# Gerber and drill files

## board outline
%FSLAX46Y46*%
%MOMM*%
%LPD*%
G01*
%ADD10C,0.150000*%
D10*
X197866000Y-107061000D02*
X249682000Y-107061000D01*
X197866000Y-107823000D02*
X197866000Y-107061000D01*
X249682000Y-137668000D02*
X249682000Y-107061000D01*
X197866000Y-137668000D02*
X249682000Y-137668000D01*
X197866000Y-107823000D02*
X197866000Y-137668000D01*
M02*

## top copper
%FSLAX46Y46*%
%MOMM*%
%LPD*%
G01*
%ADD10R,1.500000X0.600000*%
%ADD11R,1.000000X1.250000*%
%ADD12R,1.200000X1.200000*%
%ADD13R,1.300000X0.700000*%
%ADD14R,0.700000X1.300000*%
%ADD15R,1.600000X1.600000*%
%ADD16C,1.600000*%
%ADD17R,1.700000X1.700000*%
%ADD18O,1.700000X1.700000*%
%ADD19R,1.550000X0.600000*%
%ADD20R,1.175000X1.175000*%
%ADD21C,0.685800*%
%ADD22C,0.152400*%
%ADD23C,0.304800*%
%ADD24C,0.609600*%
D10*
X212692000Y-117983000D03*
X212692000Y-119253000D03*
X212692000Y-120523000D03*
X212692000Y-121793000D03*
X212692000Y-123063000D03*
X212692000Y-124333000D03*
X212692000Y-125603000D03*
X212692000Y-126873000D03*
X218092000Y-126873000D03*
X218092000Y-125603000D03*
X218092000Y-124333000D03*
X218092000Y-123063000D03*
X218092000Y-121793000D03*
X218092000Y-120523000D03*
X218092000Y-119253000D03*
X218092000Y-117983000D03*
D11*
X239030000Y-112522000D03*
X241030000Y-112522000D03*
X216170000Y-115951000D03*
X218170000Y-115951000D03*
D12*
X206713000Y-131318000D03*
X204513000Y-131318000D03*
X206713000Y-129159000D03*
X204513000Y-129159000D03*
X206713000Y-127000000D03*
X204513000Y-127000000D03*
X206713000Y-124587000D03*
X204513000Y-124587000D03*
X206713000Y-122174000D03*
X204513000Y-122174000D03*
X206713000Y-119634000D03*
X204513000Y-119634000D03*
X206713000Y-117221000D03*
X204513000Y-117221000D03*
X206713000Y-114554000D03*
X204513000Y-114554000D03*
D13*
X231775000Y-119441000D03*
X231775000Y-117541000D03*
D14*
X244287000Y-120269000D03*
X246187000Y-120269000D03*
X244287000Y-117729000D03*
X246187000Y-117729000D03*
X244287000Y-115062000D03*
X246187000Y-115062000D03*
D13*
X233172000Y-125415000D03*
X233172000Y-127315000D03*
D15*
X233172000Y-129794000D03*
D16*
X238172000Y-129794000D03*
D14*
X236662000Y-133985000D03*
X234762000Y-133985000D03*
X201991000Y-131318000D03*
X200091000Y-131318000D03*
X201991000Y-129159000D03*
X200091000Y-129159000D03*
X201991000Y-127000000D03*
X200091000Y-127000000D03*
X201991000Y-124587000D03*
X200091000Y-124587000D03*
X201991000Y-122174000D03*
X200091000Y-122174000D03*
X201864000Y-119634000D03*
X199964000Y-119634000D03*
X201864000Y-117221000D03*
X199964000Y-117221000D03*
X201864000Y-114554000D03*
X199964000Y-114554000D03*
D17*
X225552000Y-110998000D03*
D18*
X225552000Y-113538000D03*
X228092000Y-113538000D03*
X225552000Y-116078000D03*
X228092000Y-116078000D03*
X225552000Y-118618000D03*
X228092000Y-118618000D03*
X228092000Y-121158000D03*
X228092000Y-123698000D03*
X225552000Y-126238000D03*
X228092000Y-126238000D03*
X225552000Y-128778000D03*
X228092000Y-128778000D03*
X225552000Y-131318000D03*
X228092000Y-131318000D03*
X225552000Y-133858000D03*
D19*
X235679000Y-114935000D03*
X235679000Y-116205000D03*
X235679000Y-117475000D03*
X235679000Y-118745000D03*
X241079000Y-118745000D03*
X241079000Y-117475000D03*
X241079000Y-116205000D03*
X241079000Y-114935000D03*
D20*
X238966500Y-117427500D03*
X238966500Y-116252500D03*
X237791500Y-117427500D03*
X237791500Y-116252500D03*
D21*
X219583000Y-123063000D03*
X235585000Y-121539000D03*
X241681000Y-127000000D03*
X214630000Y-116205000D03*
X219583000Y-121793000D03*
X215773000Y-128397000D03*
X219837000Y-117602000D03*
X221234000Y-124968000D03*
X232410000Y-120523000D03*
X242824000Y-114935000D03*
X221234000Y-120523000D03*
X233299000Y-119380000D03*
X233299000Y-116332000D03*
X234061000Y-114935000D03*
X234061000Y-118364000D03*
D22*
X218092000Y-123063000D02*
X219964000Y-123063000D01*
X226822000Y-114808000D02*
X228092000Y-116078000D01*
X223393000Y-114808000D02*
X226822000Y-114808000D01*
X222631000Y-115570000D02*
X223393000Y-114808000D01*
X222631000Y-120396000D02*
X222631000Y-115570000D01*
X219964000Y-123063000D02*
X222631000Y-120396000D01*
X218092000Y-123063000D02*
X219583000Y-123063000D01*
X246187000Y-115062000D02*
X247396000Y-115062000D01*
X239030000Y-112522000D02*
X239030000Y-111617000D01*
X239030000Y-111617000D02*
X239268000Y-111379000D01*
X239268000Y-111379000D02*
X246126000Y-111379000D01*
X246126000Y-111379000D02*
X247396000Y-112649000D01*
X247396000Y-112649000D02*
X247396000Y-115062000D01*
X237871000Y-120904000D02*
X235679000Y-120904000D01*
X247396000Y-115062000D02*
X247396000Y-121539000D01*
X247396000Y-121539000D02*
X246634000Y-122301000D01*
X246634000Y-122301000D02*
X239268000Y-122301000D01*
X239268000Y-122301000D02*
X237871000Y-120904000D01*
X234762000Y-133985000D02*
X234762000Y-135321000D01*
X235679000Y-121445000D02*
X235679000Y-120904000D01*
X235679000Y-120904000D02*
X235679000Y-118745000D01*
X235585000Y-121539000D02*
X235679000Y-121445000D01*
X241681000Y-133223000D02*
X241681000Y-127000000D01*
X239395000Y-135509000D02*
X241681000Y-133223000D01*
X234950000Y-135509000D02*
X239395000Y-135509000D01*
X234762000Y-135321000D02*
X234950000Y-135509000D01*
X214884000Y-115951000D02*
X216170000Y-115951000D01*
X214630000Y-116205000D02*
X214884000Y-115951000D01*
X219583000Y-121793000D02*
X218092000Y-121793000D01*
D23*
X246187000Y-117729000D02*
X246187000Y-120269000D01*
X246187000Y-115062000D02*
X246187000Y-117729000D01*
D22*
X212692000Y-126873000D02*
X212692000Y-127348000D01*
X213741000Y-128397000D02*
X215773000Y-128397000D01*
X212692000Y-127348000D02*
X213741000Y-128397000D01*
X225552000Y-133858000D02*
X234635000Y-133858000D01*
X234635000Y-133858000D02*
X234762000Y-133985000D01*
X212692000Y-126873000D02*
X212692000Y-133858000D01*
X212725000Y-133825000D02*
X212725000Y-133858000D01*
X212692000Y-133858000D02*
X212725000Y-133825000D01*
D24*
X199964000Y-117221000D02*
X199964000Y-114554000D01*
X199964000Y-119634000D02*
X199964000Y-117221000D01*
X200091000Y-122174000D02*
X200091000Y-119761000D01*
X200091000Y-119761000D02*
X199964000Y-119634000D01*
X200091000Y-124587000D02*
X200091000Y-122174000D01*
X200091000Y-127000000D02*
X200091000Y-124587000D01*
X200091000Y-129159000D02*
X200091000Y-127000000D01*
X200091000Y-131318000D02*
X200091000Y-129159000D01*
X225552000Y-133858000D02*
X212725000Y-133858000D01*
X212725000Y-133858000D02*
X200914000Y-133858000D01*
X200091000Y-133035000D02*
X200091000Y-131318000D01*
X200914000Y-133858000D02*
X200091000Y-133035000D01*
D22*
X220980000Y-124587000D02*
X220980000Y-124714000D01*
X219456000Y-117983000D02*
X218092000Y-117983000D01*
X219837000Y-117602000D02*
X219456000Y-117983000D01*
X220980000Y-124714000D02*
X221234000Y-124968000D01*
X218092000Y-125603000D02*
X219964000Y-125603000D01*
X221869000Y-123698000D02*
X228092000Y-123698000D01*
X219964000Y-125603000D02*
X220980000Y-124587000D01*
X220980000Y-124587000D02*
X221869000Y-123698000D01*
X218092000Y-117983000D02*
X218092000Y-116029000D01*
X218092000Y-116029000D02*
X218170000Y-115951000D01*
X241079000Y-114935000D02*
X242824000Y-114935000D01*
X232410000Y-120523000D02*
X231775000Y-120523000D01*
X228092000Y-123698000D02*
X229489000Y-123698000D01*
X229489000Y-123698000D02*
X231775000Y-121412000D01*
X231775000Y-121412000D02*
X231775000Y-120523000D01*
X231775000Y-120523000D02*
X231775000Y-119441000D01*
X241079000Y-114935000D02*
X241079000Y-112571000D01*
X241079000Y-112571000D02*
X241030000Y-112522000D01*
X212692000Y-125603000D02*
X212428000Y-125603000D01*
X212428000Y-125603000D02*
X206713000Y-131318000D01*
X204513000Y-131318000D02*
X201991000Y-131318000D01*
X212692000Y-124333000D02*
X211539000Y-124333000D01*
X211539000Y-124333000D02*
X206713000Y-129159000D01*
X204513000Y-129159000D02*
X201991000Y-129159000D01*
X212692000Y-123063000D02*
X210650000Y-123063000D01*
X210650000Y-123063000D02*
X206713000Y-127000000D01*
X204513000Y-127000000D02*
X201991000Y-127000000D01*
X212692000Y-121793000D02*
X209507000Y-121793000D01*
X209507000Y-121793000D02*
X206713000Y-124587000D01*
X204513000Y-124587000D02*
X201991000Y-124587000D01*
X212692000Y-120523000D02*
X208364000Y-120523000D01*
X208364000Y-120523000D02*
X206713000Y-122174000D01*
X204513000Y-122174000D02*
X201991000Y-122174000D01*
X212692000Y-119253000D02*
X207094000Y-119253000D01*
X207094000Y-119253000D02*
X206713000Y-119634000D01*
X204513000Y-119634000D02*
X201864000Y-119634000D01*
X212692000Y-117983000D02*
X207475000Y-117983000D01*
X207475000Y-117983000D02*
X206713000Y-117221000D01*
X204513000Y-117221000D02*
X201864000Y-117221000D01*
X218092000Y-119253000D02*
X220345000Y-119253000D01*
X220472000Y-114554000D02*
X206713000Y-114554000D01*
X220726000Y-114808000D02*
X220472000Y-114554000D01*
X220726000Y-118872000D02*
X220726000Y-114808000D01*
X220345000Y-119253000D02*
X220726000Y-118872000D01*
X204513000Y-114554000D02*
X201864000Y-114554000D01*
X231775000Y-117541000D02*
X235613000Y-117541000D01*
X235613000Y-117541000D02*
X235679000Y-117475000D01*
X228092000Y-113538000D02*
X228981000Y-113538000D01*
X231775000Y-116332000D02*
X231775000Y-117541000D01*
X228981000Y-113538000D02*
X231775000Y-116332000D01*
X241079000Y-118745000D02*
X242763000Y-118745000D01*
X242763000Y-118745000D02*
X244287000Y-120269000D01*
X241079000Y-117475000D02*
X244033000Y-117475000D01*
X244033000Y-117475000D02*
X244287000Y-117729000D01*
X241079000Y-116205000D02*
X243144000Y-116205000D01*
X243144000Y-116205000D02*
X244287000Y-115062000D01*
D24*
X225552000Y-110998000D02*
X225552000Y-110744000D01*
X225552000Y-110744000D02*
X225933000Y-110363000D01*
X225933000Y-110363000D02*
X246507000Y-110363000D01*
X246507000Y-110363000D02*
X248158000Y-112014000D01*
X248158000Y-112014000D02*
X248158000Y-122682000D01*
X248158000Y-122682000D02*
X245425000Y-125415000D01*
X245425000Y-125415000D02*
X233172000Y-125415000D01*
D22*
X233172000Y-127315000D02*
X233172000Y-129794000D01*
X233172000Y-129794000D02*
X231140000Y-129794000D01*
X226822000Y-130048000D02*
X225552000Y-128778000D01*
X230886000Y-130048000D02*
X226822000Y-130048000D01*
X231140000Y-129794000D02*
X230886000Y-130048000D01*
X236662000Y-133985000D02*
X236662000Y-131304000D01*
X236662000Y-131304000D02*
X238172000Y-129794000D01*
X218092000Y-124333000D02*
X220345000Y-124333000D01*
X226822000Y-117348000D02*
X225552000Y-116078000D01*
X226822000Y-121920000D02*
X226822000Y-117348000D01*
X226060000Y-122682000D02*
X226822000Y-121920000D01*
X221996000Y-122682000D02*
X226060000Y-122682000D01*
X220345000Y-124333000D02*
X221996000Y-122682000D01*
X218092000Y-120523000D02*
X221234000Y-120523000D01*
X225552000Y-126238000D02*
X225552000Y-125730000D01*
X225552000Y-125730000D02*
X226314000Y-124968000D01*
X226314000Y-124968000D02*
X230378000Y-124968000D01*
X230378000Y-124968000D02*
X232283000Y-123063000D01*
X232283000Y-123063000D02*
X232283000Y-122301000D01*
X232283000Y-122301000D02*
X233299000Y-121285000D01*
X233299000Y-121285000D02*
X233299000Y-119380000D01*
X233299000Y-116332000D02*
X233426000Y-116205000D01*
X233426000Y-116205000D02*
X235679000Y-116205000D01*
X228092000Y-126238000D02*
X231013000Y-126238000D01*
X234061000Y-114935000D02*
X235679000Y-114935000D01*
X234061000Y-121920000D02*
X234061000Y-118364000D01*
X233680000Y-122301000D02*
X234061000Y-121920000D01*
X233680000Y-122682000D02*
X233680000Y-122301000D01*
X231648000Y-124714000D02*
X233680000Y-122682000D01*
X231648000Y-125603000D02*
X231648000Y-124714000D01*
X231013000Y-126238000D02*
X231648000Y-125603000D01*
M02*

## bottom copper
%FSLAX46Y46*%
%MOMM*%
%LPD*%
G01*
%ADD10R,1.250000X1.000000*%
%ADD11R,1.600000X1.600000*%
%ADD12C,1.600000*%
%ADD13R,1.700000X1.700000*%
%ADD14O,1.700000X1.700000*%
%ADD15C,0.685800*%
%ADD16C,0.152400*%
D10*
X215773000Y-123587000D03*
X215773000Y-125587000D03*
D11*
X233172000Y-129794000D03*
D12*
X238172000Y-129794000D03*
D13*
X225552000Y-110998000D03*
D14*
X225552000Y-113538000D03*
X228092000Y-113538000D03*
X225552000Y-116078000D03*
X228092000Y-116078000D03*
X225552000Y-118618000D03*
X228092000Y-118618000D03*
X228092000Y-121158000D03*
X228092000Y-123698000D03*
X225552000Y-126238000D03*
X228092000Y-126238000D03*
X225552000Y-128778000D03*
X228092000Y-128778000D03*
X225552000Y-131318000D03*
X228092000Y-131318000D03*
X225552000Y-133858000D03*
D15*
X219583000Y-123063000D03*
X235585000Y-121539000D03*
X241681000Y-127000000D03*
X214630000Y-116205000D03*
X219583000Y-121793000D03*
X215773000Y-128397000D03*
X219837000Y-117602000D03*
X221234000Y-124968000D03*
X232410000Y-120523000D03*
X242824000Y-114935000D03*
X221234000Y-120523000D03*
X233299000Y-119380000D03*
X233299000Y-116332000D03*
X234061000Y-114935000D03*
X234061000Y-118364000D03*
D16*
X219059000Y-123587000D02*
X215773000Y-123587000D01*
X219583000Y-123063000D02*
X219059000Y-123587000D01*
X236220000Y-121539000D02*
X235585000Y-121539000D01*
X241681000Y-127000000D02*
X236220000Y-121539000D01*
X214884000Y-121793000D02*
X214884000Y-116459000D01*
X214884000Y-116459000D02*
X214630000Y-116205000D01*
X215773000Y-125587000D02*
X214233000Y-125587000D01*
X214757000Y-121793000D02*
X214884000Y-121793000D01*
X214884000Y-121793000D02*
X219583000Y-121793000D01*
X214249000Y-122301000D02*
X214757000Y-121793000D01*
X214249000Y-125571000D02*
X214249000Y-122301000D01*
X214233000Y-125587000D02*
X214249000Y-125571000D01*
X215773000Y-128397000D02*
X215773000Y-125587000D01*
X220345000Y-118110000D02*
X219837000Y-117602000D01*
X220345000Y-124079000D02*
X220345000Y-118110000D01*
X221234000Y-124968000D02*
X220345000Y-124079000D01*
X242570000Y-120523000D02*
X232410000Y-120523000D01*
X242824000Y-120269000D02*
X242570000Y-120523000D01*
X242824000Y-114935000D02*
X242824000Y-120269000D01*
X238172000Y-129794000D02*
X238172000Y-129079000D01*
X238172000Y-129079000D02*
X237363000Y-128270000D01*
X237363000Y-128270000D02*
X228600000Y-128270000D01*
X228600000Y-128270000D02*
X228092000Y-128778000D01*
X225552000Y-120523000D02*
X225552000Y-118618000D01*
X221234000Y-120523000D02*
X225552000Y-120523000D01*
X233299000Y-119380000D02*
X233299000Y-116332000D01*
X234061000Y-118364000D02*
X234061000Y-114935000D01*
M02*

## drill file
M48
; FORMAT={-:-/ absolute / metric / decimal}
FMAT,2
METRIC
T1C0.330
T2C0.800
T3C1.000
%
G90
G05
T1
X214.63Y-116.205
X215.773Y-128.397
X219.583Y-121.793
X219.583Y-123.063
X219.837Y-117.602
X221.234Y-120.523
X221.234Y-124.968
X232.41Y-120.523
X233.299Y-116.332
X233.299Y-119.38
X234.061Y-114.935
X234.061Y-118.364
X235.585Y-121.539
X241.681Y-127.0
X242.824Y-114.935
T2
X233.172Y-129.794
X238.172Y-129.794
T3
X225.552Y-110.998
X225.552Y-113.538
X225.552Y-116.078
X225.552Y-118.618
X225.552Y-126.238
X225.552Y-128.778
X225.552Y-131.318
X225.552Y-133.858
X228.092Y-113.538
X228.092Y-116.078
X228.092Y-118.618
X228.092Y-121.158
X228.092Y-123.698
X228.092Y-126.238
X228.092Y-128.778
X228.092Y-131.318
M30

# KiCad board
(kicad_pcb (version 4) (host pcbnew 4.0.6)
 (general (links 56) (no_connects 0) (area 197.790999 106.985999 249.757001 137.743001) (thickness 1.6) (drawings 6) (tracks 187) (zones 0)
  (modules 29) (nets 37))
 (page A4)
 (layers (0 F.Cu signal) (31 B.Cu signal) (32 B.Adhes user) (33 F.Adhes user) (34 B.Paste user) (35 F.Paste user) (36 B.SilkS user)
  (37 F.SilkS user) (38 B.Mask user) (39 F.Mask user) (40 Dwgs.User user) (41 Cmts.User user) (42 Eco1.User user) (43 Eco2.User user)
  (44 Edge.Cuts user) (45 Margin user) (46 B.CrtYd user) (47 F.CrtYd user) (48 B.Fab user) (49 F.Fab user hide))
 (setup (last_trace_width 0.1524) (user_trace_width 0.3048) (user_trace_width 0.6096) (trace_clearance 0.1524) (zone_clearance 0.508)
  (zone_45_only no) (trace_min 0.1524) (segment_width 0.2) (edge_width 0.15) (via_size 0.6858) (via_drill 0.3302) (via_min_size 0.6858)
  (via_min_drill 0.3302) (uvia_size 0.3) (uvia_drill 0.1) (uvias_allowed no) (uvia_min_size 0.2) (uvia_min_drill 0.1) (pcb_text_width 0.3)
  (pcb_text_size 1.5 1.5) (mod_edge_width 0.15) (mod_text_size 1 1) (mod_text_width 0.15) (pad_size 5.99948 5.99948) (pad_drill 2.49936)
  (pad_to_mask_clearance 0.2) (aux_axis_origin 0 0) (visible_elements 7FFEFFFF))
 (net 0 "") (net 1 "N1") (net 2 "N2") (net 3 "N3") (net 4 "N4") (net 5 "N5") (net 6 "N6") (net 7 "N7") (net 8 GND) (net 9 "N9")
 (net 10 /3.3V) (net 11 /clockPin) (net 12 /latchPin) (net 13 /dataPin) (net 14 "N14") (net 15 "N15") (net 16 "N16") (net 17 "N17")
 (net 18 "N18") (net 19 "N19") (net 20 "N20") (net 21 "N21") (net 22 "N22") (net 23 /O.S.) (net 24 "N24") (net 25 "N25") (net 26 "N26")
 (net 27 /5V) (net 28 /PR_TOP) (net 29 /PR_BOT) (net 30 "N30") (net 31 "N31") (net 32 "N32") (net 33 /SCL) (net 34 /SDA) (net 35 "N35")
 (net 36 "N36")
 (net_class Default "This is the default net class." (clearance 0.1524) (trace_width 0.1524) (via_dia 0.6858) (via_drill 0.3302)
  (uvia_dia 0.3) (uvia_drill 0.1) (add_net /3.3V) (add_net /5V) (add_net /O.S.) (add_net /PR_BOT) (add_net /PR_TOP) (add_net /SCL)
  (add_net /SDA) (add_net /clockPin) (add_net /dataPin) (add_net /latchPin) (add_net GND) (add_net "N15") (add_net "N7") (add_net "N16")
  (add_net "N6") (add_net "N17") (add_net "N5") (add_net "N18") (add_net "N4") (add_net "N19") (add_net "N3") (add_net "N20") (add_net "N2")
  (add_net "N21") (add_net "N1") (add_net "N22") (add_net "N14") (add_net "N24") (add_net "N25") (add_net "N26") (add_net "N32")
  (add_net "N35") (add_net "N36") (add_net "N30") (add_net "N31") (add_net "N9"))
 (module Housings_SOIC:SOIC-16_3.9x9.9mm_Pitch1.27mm (layer F.Cu) (at 215.392 122.428)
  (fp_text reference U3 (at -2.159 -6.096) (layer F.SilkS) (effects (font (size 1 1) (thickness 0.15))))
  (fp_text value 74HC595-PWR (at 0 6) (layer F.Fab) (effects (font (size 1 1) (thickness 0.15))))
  (pad 1 smd rect (at -2.7 -4.445) (size 1.5 0.6) (layers F.Cu F.Paste F.Mask) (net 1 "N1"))
  (pad 2 smd rect (at -2.7 -3.175) (size 1.5 0.6) (layers F.Cu F.Paste F.Mask) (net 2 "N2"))
  (pad 3 smd rect (at -2.7 -1.905) (size 1.5 0.6) (layers F.Cu F.Paste F.Mask) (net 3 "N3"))
  (pad 4 smd rect (at -2.7 -0.635) (size 1.5 0.6) (layers F.Cu F.Paste F.Mask) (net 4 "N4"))
  (pad 5 smd rect (at -2.7 0.635) (size 1.5 0.6) (layers F.Cu F.Paste F.Mask) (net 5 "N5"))
  (pad 6 smd rect (at -2.7 1.905) (size 1.5 0.6) (layers F.Cu F.Paste F.Mask) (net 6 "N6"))
  (pad 7 smd rect (at -2.7 3.175) (size 1.5 0.6) (layers F.Cu F.Paste F.Mask) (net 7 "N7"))
  (pad 8 smd rect (at -2.7 4.445) (size 1.5 0.6) (layers F.Cu F.Paste F.Mask) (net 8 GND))
  (pad 9 smd rect (at 2.7 4.445) (size 1.5 0.6) (layers F.Cu F.Paste F.Mask) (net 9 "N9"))
  (pad 10 smd rect (at 2.7 3.175) (size 1.5 0.6) (layers F.Cu F.Paste F.Mask) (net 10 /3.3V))
  (pad 11 smd rect (at 2.7 1.905) (size 1.5 0.6) (layers F.Cu F.Paste F.Mask) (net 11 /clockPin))
  (pad 12 smd rect (at 2.7 0.635) (size 1.5 0.6) (layers F.Cu F.Paste F.Mask) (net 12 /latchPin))
  (pad 13 smd rect (at 2.7 -0.635) (size 1.5 0.6) (layers F.Cu F.Paste F.Mask) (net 8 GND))
  (pad 14 smd rect (at 2.7 -1.905) (size 1.5 0.6) (layers F.Cu F.Paste F.Mask) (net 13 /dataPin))
  (pad 15 smd rect (at 2.7 -3.175) (size 1.5 0.6) (layers F.Cu F.Paste F.Mask) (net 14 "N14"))
  (pad 16 smd rect (at 2.7 -4.445) (size 1.5 0.6) (layers F.Cu F.Paste F.Mask) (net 10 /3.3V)))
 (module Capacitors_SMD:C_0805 (layer B.Cu) (at 215.773 124.587 270)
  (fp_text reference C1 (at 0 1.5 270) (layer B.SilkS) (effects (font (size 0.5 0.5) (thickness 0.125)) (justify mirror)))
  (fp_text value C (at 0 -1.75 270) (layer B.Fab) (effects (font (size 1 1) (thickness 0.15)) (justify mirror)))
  (pad 1 smd rect (at -1 0 270) (size 1 1.25) (layers B.Cu B.Paste B.Mask) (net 12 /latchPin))
  (pad 2 smd rect (at 1 0 270) (size 1 1.25) (layers B.Cu B.Paste B.Mask) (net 8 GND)))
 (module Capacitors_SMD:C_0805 (layer F.Cu) (at 240.03 112.522)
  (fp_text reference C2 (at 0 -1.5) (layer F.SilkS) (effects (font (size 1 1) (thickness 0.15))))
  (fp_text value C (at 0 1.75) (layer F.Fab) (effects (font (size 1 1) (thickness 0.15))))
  (pad 1 smd rect (at -1 0) (size 1 1.25) (layers F.Cu F.Paste F.Mask) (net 8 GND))
  (pad 2 smd rect (at 1 0) (size 1 1.25) (layers F.Cu F.Paste F.Mask) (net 10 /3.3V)))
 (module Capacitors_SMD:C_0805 (layer F.Cu) (at 217.17 115.951)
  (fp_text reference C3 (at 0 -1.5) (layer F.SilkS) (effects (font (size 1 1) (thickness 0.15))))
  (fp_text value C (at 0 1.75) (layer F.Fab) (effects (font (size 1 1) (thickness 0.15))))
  (pad 1 smd rect (at -1 0) (size 1 1.25) (layers F.Cu F.Paste F.Mask) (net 8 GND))
  (pad 2 smd rect (at 1 0) (size 1 1.25) (layers F.Cu F.Paste F.Mask) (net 10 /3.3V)))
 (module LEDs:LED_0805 (layer F.Cu) (at 205.613 131.318)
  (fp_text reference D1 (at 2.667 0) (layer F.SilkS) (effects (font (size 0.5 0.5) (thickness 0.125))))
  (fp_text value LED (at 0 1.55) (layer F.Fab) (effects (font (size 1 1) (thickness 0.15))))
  (pad 2 smd rect (at 1.1 0 180) (size 1.2 1.2) (layers F.Cu F.Paste F.Mask) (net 7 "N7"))
  (pad 1 smd rect (at -1.1 0 180) (size 1.2 1.2) (layers F.Cu F.Paste F.Mask) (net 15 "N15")))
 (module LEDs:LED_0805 (layer F.Cu) (at 205.613 129.159)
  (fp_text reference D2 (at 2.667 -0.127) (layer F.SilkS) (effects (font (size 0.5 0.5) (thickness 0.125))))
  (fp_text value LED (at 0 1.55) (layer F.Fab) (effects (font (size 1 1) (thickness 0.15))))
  (pad 2 smd rect (at 1.1 0 180) (size 1.2 1.2) (layers F.Cu F.Paste F.Mask) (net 6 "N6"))
  (pad 1 smd rect (at -1.1 0 180) (size 1.2 1.2) (layers F.Cu F.Paste F.Mask) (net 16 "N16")))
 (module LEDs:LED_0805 (layer F.Cu) (at 205.613 127)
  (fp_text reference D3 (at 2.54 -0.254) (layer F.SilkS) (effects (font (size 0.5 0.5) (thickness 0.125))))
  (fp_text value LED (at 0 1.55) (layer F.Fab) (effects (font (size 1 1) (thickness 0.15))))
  (pad 2 smd rect (at 1.1 0 180) (size 1.2 1.2) (layers F.Cu F.Paste F.Mask) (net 5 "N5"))
  (pad 1 smd rect (at -1.1 0 180) (size 1.2 1.2) (layers F.Cu F.Paste F.Mask) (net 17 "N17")))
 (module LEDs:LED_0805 (layer F.Cu) (at 205.613 124.587)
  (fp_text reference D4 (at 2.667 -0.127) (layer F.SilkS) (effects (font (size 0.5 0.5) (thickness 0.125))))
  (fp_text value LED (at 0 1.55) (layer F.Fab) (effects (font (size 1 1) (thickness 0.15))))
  (pad 2 smd rect (at 1.1 0 180) (size 1.2 1.2) (layers F.Cu F.Paste F.Mask) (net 4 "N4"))
  (pad 1 smd rect (at -1.1 0 180) (size 1.2 1.2) (layers F.Cu F.Paste F.Mask) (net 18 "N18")))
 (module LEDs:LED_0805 (layer F.Cu) (at 205.613 122.174)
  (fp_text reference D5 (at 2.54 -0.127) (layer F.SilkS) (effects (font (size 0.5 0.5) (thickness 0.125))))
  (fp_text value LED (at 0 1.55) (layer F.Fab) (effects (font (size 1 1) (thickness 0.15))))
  (pad 2 smd rect (at 1.1 0 180) (size 1.2 1.2) (layers F.Cu F.Paste F.Mask) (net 3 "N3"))
  (pad 1 smd rect (at -1.1 0 180) (size 1.2 1.2) (layers F.Cu F.Paste F.Mask) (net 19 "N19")))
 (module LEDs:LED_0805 (layer F.Cu) (at 205.613 119.634)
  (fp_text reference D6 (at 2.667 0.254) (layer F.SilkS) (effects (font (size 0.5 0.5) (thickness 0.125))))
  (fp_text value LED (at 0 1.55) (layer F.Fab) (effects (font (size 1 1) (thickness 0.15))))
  (pad 2 smd rect (at 1.1 0 180) (size 1.2 1.2) (layers F.Cu F.Paste F.Mask) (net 2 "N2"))
  (pad 1 smd rect (at -1.1 0 180) (size 1.2 1.2) (layers F.Cu F.Paste F.Mask) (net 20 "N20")))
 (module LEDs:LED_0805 (layer F.Cu) (at 205.613 117.221)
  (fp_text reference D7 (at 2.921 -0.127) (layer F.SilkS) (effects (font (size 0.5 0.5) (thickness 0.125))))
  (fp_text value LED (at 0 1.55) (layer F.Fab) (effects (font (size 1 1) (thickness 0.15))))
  (pad 2 smd rect (at 1.1 0 180) (size 1.2 1.2) (layers F.Cu F.Paste F.Mask) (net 1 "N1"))
  (pad 1 smd rect (at -1.1 0 180) (size 1.2 1.2) (layers F.Cu F.Paste F.Mask) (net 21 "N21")))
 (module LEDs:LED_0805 (layer F.Cu) (at 205.613 114.554)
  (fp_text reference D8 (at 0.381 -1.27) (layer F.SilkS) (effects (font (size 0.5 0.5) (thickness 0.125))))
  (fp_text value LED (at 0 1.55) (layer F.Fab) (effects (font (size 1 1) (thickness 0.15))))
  (pad 2 smd rect (at 1.1 0 180) (size 1.2 1.2) (layers F.Cu F.Paste F.Mask) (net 14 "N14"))
  (pad 1 smd rect (at -1.1 0 180) (size 1.2 1.2) (layers F.Cu F.Paste F.Mask) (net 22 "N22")))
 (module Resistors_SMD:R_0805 (layer F.Cu) (at 231.775 118.491 90)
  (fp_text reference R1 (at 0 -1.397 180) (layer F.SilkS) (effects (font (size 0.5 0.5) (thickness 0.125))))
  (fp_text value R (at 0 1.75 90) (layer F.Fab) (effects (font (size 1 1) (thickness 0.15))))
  (pad 1 smd rect (at -0.95 0 90) (size 0.7 1.3) (layers F.Cu F.Paste F.Mask) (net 10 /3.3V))
  (pad 2 smd rect (at 0.95 0 90) (size 0.7 1.3) (layers F.Cu F.Paste F.Mask) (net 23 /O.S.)))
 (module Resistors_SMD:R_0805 (layer F.Cu) (at 245.237 120.269)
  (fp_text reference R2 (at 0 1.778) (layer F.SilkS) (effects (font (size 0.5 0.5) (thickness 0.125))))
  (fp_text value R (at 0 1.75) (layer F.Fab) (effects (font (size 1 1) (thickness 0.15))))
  (pad 1 smd rect (at -0.95 0) (size 0.7 1.3) (layers F.Cu F.Paste F.Mask) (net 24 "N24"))
  (pad 2 smd rect (at 0.95 0) (size 0.7 1.3) (layers F.Cu F.Paste F.Mask) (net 8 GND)))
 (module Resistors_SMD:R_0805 (layer F.Cu) (at 245.237 117.729)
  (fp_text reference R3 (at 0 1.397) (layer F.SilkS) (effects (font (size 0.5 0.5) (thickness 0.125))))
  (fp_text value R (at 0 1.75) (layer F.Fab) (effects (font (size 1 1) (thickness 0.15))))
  (pad 1 smd rect (at -0.95 0) (size 0.7 1.3) (layers F.Cu F.Paste F.Mask) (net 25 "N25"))
  (pad 2 smd rect (at 0.95 0) (size 0.7 1.3) (layers F.Cu F.Paste F.Mask) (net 8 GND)))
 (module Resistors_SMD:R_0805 (layer F.Cu) (at 245.237 115.062)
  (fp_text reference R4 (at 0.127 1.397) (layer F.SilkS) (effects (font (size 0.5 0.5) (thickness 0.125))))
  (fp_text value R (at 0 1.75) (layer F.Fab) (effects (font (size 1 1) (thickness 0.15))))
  (pad 1 smd rect (at -0.95 0) (size 0.7 1.3) (layers F.Cu F.Paste F.Mask) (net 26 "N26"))
  (pad 2 smd rect (at 0.95 0) (size 0.7 1.3) (layers F.Cu F.Paste F.Mask) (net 8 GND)))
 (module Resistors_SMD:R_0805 (layer F.Cu) (at 233.172 126.365 270)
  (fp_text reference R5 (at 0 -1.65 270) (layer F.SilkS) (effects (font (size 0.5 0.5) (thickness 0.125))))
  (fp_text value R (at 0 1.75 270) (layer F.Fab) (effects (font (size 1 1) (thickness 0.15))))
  (pad 1 smd rect (at -0.95 0 270) (size 0.7 1.3) (layers F.Cu F.Paste F.Mask) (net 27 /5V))
  (pad 2 smd rect (at 0.95 0 270) (size 0.7 1.3) (layers F.Cu F.Paste F.Mask) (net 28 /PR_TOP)))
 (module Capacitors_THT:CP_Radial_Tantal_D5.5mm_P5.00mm (layer F.Cu) (at 233.172 129.794)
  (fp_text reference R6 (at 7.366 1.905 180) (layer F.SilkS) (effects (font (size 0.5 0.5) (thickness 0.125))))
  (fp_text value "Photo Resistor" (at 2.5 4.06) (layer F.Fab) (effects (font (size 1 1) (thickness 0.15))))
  (pad 1 thru_hole rect (at 0 0) (size 1.6 1.6) (drill 0.8) (layers *.Cu *.Mask) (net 28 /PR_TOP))
  (pad 2 thru_hole circle (at 5 0) (size 1.6 1.6) (drill 0.8) (layers *.Cu *.Mask) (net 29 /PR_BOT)))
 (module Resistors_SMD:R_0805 (layer F.Cu) (at 235.712 133.985 180)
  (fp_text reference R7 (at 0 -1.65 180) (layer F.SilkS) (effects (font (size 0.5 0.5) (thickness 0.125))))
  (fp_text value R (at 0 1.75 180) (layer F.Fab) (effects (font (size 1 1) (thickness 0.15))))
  (pad 1 smd rect (at -0.95 0 180) (size 0.7 1.3) (layers F.Cu F.Paste F.Mask) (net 29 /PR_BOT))
  (pad 2 smd rect (at 0.95 0 180) (size 0.7 1.3) (layers F.Cu F.Paste F.Mask) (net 8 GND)))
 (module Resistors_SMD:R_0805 (layer F.Cu) (at 201.041 131.318 180)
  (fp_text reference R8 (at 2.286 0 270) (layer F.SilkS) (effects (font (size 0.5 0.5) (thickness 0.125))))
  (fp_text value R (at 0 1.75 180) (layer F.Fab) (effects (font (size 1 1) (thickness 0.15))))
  (pad 1 smd rect (at -0.95 0 180) (size 0.7 1.3) (layers F.Cu F.Paste F.Mask) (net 15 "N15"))
  (pad 2 smd rect (at 0.95 0 180) (size 0.7 1.3) (layers F.Cu F.Paste F.Mask) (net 8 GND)))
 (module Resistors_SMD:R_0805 (layer F.Cu) (at 201.041 129.159 180)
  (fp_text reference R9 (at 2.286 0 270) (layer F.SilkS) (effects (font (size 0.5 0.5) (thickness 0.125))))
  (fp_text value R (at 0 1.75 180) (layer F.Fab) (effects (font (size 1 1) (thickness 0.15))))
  (pad 1 smd rect (at -0.95 0 180) (size 0.7 1.3) (layers F.Cu F.Paste F.Mask) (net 16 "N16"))
  (pad 2 smd rect (at 0.95 0 180) (size 0.7 1.3) (layers F.Cu F.Paste F.Mask) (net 8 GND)))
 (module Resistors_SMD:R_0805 (layer F.Cu) (at 201.041 127 180)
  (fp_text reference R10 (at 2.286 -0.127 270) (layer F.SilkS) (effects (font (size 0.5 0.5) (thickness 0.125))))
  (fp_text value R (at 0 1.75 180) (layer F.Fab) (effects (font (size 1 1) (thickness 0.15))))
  (pad 1 smd rect (at -0.95 0 180) (size 0.7 1.3) (layers F.Cu F.Paste F.Mask) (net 17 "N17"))
  (pad 2 smd rect (at 0.95 0 180) (size 0.7 1.3) (layers F.Cu F.Paste F.Mask) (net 8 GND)))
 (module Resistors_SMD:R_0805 (layer F.Cu) (at 201.041 124.587 180)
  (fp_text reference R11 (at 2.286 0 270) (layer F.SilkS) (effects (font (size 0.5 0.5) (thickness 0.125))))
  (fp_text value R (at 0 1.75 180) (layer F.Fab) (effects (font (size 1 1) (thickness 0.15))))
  (pad 1 smd rect (at -0.95 0 180) (size 0.7 1.3) (layers F.Cu F.Paste F.Mask) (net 18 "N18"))
  (pad 2 smd rect (at 0.95 0 180) (size 0.7 1.3) (layers F.Cu F.Paste F.Mask) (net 8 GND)))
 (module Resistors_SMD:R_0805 (layer F.Cu) (at 201.041 122.174 180)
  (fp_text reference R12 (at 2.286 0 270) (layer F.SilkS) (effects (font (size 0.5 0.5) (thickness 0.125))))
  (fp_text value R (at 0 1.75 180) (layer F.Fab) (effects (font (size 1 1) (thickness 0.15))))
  (pad 1 smd rect (at -0.95 0 180) (size 0.7 1.3) (layers F.Cu F.Paste F.Mask) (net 19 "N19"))
  (pad 2 smd rect (at 0.95 0 180) (size 0.7 1.3) (layers F.Cu F.Paste F.Mask) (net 8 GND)))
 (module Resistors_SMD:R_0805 (layer F.Cu) (at 200.914 119.634 180)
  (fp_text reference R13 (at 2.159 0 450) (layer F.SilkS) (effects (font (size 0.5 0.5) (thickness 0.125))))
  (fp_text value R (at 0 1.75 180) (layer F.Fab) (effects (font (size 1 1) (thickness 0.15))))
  (pad 1 smd rect (at -0.95 0 180) (size 0.7 1.3) (layers F.Cu F.Paste F.Mask) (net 20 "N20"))
  (pad 2 smd rect (at 0.95 0 180) (size 0.7 1.3) (layers F.Cu F.Paste F.Mask) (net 8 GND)))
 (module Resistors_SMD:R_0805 (layer F.Cu) (at 200.914 117.221 180)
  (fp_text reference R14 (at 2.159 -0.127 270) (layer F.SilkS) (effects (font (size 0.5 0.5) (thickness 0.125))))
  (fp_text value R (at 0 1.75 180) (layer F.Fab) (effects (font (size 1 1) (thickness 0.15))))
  (pad 1 smd rect (at -0.95 0 180) (size 0.7 1.3) (layers F.Cu F.Paste F.Mask) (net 21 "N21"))
  (pad 2 smd rect (at 0.95 0 180) (size 0.7 1.3) (layers F.Cu F.Paste F.Mask) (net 8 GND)))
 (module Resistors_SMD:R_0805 (layer F.Cu) (at 200.914 114.554 180)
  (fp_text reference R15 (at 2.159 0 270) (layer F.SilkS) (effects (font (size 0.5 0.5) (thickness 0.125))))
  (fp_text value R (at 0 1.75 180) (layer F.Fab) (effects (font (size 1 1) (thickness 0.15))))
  (pad 1 smd rect (at -0.95 0 180) (size 0.7 1.3) (layers F.Cu F.Paste F.Mask) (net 22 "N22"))
  (pad 2 smd rect (at 0.95 0 180) (size 0.7 1.3) (layers F.Cu F.Paste F.Mask) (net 8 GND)))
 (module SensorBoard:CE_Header (layer F.Cu) (at 225.552 110.998)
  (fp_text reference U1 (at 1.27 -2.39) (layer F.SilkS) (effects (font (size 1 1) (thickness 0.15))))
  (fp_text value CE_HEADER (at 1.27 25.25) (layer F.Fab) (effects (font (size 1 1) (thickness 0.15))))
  (pad 1 thru_hole rect (at 0 0) (size 1.7 1.7) (drill 1) (layers *.Cu *.Mask) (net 27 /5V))
  (pad 3 thru_hole oval (at 0 2.54) (size 1.7 1.7) (drill 1) (layers *.Cu *.Mask) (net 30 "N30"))
  (pad 4 thru_hole oval (at 2.54 2.54) (size 1.7 1.7) (drill 1) (layers *.Cu *.Mask) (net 23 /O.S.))
  (pad 5 thru_hole oval (at 0 5.08) (size 1.7 1.7) (drill 1) (layers *.Cu *.Mask) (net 11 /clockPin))
  (pad 6 thru_hole oval (at 2.54 5.08) (size 1.7 1.7) (drill 1) (layers *.Cu *.Mask) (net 12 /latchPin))
  (pad 7 thru_hole oval (at 0 7.62) (size 1.7 1.7) (drill 1) (layers *.Cu *.Mask) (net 13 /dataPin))
  (pad 8 thru_hole oval (at 2.54 7.62) (size 1.7 1.7) (drill 1) (layers *.Cu *.Mask) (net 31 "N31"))
  (pad 10 thru_hole oval (at 2.54 10.16) (size 1.7 1.7) (drill 1) (layers *.Cu *.Mask) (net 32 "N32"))
  (pad 12 thru_hole oval (at 2.54 12.7) (size 1.7 1.7) (drill 1) (layers *.Cu *.Mask) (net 10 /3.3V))
  (pad 13 thru_hole oval (at 0 15.24) (size 1.7 1.7) (drill 1) (layers *.Cu *.Mask) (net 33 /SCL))
  (pad 14 thru_hole oval (at 2.54 15.24) (size 1.7 1.7) (drill 1) (layers *.Cu *.Mask) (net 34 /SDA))
  (pad 15 thru_hole oval (at 0 17.78) (size 1.7 1.7) (drill 1) (layers *.Cu *.Mask) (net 28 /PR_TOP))
  (pad 16 thru_hole oval (at 2.54 17.78) (size 1.7 1.7) (drill 1) (layers *.Cu *.Mask) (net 29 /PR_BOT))
  (pad 17 thru_hole oval (at 0 20.32) (size 1.7 1.7) (drill 1) (layers *.Cu *.Mask) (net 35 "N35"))
  (pad 18 thru_hole oval (at 2.54 20.32) (size 1.7 1.7) (drill 1) (layers *.Cu *.Mask) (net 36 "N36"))
  (pad 19 thru_hole oval (at 0 22.86) (size 1.7 1.7) (drill 1) (layers *.Cu *.Mask) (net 8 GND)))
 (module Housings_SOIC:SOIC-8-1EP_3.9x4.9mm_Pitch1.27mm (layer F.Cu) (at 238.379 116.84)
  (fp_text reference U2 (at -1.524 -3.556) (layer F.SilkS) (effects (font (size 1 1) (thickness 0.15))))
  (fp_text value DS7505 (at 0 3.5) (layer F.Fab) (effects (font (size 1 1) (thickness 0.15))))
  (pad 1 smd rect (at -2.7 -1.905) (size 1.55 0.6) (layers F.Cu F.Paste F.Mask) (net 34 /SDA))
  (pad 2 smd rect (at -2.7 -0.635) (size 1.55 0.6) (layers F.Cu F.Paste F.Mask) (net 33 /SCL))
  (pad 3 smd rect (at -2.7 0.635) (size 1.55 0.6) (layers F.Cu F.Paste F.Mask) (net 23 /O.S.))
  (pad 4 smd rect (at -2.7 1.905) (size 1.55 0.6) (layers F.Cu F.Paste F.Mask) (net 8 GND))
  (pad 5 smd rect (at 2.7 1.905) (size 1.55 0.6) (layers F.Cu F.Paste F.Mask) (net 24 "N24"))
  (pad 6 smd rect (at 2.7 0.635) (size 1.55 0.6) (layers F.Cu F.Paste F.Mask) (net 25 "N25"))
  (pad 7 smd rect (at 2.7 -0.635) (size 1.55 0.6) (layers F.Cu F.Paste F.Mask) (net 26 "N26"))
  (pad 8 smd rect (at 2.7 -1.905) (size 1.55 0.6) (layers F.Cu F.Paste F.Mask) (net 10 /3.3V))
  (pad 9 smd rect (at 0.5875 0.5875) (size 1.175 1.175) (layers F.Cu F.Paste F.Mask) (solder_paste_margin_ratio -0.2))
  (pad 9 smd rect (at 0.5875 -0.5875) (size 1.175 1.175) (layers F.Cu F.Paste F.Mask) (solder_paste_margin_ratio -0.2))
  (pad 9 smd rect (at -0.5875 0.5875) (size 1.175 1.175) (layers F.Cu F.Paste F.Mask) (solder_paste_margin_ratio -0.2))
  (pad 9 smd rect (at -0.5875 -0.5875) (size 1.175 1.175) (layers F.Cu F.Paste F.Mask) (solder_paste_margin_ratio -0.2)))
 (gr_line (start 197.866 107.061) (end 249.682 107.061) (angle 90) (layer Edge.Cuts) (width 0.15))
 (gr_line (start 197.866 107.823) (end 197.866 107.061) (angle 90) (layer Edge.Cuts) (width 0.15))
 (gr_line (start 249.682 137.668) (end 249.682 107.061) (angle 90) (layer Edge.Cuts) (width 0.15))
 (gr_line (start 197.866 137.668) (end 249.682 137.668) (angle 90) (layer Edge.Cuts) (width 0.15))
 (gr_line (start 197.866 107.823) (end 197.866 137.668) (angle 90) (layer Edge.Cuts) (width 0.15))
 (segment (start 218.092 123.063) (end 219.964 123.063) (width 0.1524) (layer F.Cu) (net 12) (status 10))
 (segment (start 226.822 114.808) (end 228.092 116.078) (width 0.1524) (layer F.Cu) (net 12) (status 20))
 (segment (start 223.393 114.808) (end 226.822 114.808) (width 0.1524) (layer F.Cu) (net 12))
 (segment (start 222.631 115.57) (end 223.393 114.808) (width 0.1524) (layer F.Cu) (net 12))
 (segment (start 222.631 120.396) (end 222.631 115.57) (width 0.1524) (layer F.Cu) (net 12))
 (segment (start 219.964 123.063) (end 222.631 120.396) (width 0.1524) (layer F.Cu) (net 12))
 (segment (start 218.092 123.063) (end 219.583 123.063) (width 0.1524) (layer F.Cu) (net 12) (status 10))
 (segment (start 219.059 123.587) (end 215.773 123.587) (width 0.1524) (layer B.Cu) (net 12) (status 20))
 (segment (start 219.583 123.063) (end 219.059 123.587) (width 0.1524) (layer B.Cu) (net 12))
 (via (at 219.583 123.063) (size 0.6858) (drill 0.3302) (layers F.Cu B.Cu) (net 12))
 (segment (start 246.187 115.062) (end 247.396 115.062) (width 0.1524) (layer F.Cu) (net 8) (status 10))
 (segment (start 239.03 112.522) (end 239.03 111.617) (width 0.1524) (layer F.Cu) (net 8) (status 10))
 (segment (start 239.03 111.617) (end 239.268 111.379) (width 0.1524) (layer F.Cu) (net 8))
 (segment (start 239.268 111.379) (end 246.126 111.379) (width 0.1524) (layer F.Cu) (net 8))
 (segment (start 246.126 111.379) (end 247.396 112.649) (width 0.1524) (layer F.Cu) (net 8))
 (segment (start 247.396 112.649) (end 247.396 115.062) (width 0.1524) (layer F.Cu) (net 8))
 (segment (start 237.871 120.904) (end 235.679 120.904) (width 0.1524) (layer F.Cu) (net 8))
 (segment (start 247.396 115.062) (end 247.396 121.539) (width 0.1524) (layer F.Cu) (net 8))
 (segment (start 247.396 121.539) (end 246.634 122.301) (width 0.1524) (layer F.Cu) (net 8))
 (segment (start 246.634 122.301) (end 239.268 122.301) (width 0.1524) (layer F.Cu) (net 8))
 (segment (start 239.268 122.301) (end 237.871 120.904) (width 0.1524) (layer F.Cu) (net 8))
 (segment (start 234.762 133.985) (end 234.762 135.321) (width 0.1524) (layer F.Cu) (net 8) (status 10))
 (segment (start 235.679 121.445) (end 235.679 120.904) (width 0.1524) (layer F.Cu) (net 8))
 (segment (start 235.679 120.904) (end 235.679 118.745) (width 0.1524) (layer F.Cu) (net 8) (status 20))
 (segment (start 235.585 121.539) (end 235.679 121.445) (width 0.1524) (layer F.Cu) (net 8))
 (via (at 235.585 121.539) (size 0.6858) (drill 0.3302) (layers F.Cu B.Cu) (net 8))
 (segment (start 236.22 121.539) (end 235.585 121.539) (width 0.1524) (layer B.Cu) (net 8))
 (segment (start 241.681 127) (end 236.22 121.539) (width 0.1524) (layer B.Cu) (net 8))
 (via (at 241.681 127) (size 0.6858) (drill 0.3302) (layers F.Cu B.Cu) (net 8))
 (segment (start 241.681 133.223) (end 241.681 127) (width 0.1524) (layer F.Cu) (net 8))
 (segment (start 239.395 135.509) (end 241.681 133.223) (width 0.1524) (layer F.Cu) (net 8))
 (segment (start 234.95 135.509) (end 239.395 135.509) (width 0.1524) (layer F.Cu) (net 8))
 (segment (start 234.762 135.321) (end 234.95 135.509) (width 0.1524) (layer F.Cu) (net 8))
 (segment (start 214.884 121.793) (end 214.884 116.459) (width 0.1524) (layer B.Cu) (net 8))
 (segment (start 214.884 115.951) (end 216.17 115.951) (width 0.1524) (layer F.Cu) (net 8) (status 20))
 (segment (start 214.63 116.205) (end 214.884 115.951) (width 0.1524) (layer F.Cu) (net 8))
 (via (at 214.63 116.205) (size 0.6858) (drill 0.3302) (layers F.Cu B.Cu) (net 8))
 (segment (start 214.884 116.459) (end 214.63 116.205) (width 0.1524) (layer B.Cu) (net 8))
 (segment (start 215.773 125.587) (end 214.233 125.587) (width 0.1524) (layer B.Cu) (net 8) (status 10))
 (segment (start 219.583 121.793) (end 218.092 121.793) (width 0.1524) (layer F.Cu) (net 8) (status 20))
 (via (at 219.583 121.793) (size 0.6858) (drill 0.3302) (layers F.Cu B.Cu) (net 8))
 (segment (start 214.757 121.793) (end 214.884 121.793) (width 0.1524) (layer B.Cu) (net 8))
 (segment (start 214.884 121.793) (end 219.583 121.793) (width 0.1524) (layer B.Cu) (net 8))
 (segment (start 214.249 122.301) (end 214.757 121.793) (width 0.1524) (layer B.Cu) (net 8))
 (segment (start 214.249 125.571) (end 214.249 122.301) (width 0.1524) (layer B.Cu) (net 8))
 (segment (start 214.233 125.587) (end 214.249 125.571) (width 0.1524) (layer B.Cu) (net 8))
 (segment (start 246.187 117.729) (end 246.187 120.269) (width 0.3048) (layer F.Cu) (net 8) (status 30))
 (segment (start 246.187 115.062) (end 246.187 117.729) (width 0.3048) (layer F.Cu) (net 8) (status 30))
 (segment (start 212.692 126.873) (end 212.692 127.348) (width 0.1524) (layer F.Cu) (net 8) (status 10))
 (segment (start 215.773 128.397) (end 215.773 125.587) (width 0.1524) (layer B.Cu) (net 8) (status 20))
 (via (at 215.773 128.397) (size 0.6858) (drill 0.3302) (layers F.Cu B.Cu) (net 8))
 (segment (start 213.741 128.397) (end 215.773 128.397) (width 0.1524) (layer F.Cu) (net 8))
 (segment (start 212.692 127.348) (end 213.741 128.397) (width 0.1524) (layer F.Cu) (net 8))
 (segment (start 225.552 133.858) (end 234.635 133.858) (width 0.1524) (layer F.Cu) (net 8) (status 30))
 (segment (start 234.635 133.858) (end 234.762 133.985) (width 0.1524) (layer F.Cu) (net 8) (status 30))
 (segment (start 212.692 126.873) (end 212.692 133.858) (width 0.1524) (layer F.Cu) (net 8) (status 10))
 (segment (start 212.725 133.825) (end 212.725 133.858) (width 0.1524) (layer F.Cu) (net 8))
 (segment (start 212.692 133.858) (end 212.725 133.825) (width 0.1524) (layer F.Cu) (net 8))
 (segment (start 199.964 117.221) (end 199.964 114.554) (width 0.6096) (layer F.Cu) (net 8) (status 30))
 (segment (start 199.964 119.634) (end 199.964 117.221) (width 0.6096) (layer F.Cu) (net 8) (status 30))
 (segment (start 200.091 122.174) (end 200.091 119.761) (width 0.6096) (layer F.Cu) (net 8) (status 30))
 (segment (start 200.091 119.761) (end 199.964 119.634) (width 0.6096) (layer F.Cu) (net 8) (status 30))
 (segment (start 200.091 124.587) (end 200.091 122.174) (width 0.6096) (layer F.Cu) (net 8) (status 30))
 (segment (start 200.091 127) (end 200.091 124.587) (width 0.6096) (layer F.Cu) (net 8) (status 30))
 (segment (start 200.091 129.159) (end 200.091 127) (width 0.6096) (layer F.Cu) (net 8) (status 30))
 (segment (start 200.091 131.318) (end 200.091 129.159) (width 0.6096) (layer F.Cu) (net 8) (status 30))
 (segment (start 225.552 133.858) (end 212.725 133.858) (width 0.6096) (layer F.Cu) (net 8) (status 10))
 (segment (start 212.725 133.858) (end 200.914 133.858) (width 0.6096) (layer F.Cu) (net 8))
 (segment (start 200.091 133.035) (end 200.091 131.318) (width 0.6096) (layer F.Cu) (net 8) (status 20))
 (segment (start 200.914 133.858) (end 200.091 133.035) (width 0.6096) (layer F.Cu) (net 8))
 (segment (start 220.98 124.587) (end 220.98 124.714) (width 0.1524) (layer F.Cu) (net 10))
 (segment (start 219.456 117.983) (end 218.092 117.983) (width 0.1524) (layer F.Cu) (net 10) (status 20))
 (segment (start 219.837 117.602) (end 219.456 117.983) (width 0.1524) (layer F.Cu) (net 10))
 (via (at 219.837 117.602) (size 0.6858) (drill 0.3302) (layers F.Cu B.Cu) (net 10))
 (segment (start 220.345 118.11) (end 219.837 117.602) (width 0.1524) (layer B.Cu) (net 10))
 (segment (start 220.345 124.079) (end 220.345 118.11) (width 0.1524) (layer B.Cu) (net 10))
 (segment (start 221.234 124.968) (end 220.345 124.079) (width 0.1524) (layer B.Cu) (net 10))
 (via (at 221.234 124.968) (size 0.6858) (drill 0.3302) (layers F.Cu B.Cu) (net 10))
 (segment (start 220.98 124.714) (end 221.234 124.968) (width 0.1524) (layer F.Cu) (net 10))
 (segment (start 218.092 125.603) (end 219.964 125.603) (width 0.1524) (layer F.Cu) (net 10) (status 10))
 (segment (start 221.869 123.698) (end 228.092 123.698) (width 0.1524) (layer F.Cu) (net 10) (status 20))
 (segment (start 219.964 125.603) (end 220.98 124.587) (width 0.1524) (layer F.Cu) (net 10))
 (segment (start 220.98 124.587) (end 221.869 123.698) (width 0.1524) (layer F.Cu) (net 10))
 (segment (start 218.092 117.983) (end 218.092 116.029) (width 0.1524) (layer F.Cu) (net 10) (status 20))
 (segment (start 218.092 116.029) (end 218.17 115.951) (width 0.1524) (layer F.Cu) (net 10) (status 30))
 (segment (start 241.079 114.935) (end 242.824 114.935) (width 0.1524) (layer F.Cu) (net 10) (status 10))
 (segment (start 232.41 120.523) (end 231.775 120.523) (width 0.1524) (layer F.Cu) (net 10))
 (via (at 232.41 120.523) (size 0.6858) (drill 0.3302) (layers F.Cu B.Cu) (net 10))
 (segment (start 242.57 120.523) (end 232.41 120.523) (width 0.1524) (layer B.Cu) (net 10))
 (segment (start 242.824 120.269) (end 242.57 120.523) (width 0.1524) (layer B.Cu) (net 10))
 (segment (start 242.824 114.935) (end 242.824 120.269) (width 0.1524) (layer B.Cu) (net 10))
 (via (at 242.824 114.935) (size 0.6858) (drill 0.3302) (layers F.Cu B.Cu) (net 10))
 (segment (start 228.092 123.698) (end 229.489 123.698) (width 0.1524) (layer F.Cu) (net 10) (status 10))
 (segment (start 229.489 123.698) (end 231.775 121.412) (width 0.1524) (layer F.Cu) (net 10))
 (segment (start 231.775 121.412) (end 231.775 120.523) (width 0.1524) (layer F.Cu) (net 10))
 (segment (start 231.775 120.523) (end 231.775 119.441) (width 0.1524) (layer F.Cu) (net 10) (status 20))
 (segment (start 241.079 114.935) (end 241.079 112.571) (width 0.1524) (layer F.Cu) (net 10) (status 30))
 (segment (start 241.079 112.571) (end 241.03 112.522) (width 0.1524) (layer F.Cu) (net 10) (status 30))
 (segment (start 212.692 125.603) (end 212.428 125.603) (width 0.1524) (layer F.Cu) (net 7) (status 30))
 (segment (start 212.428 125.603) (end 206.713 131.318) (width 0.1524) (layer F.Cu) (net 7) (status 30))
 (segment (start 204.513 131.318) (end 201.991 131.318) (width 0.1524) (layer F.Cu) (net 15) (status 30))
 (segment (start 212.692 124.333) (end 211.539 124.333) (width 0.1524) (layer F.Cu) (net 6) (status 10))
 (segment (start 211.539 124.333) (end 206.713 129.159) (width 0.1524) (layer F.Cu) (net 6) (status 20))
 (segment (start 204.513 129.159) (end 201.991 129.159) (width 0.1524) (layer F.Cu) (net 16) (status 30))
 (segment (start 212.692 123.063) (end 210.65 123.063) (width 0.1524) (layer F.Cu) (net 5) (status 10))
 (segment (start 210.65 123.063) (end 206.713 127) (width 0.1524) (layer F.Cu) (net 5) (status 20))
 (segment (start 204.513 127) (end 201.991 127) (width 0.1524) (layer F.Cu) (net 17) (status 30))
 (segment (start 212.692 121.793) (end 209.507 121.793) (width 0.1524) (layer F.Cu) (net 4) (status 10))
 (segment (start 209.507 121.793) (end 206.713 124.587) (width 0.1524) (layer F.Cu) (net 4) (status 20))
 (segment (start 204.513 124.587) (end 201.991 124.587) (width 0.1524) (layer F.Cu) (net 18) (status 30))
 (segment (start 212.692 120.523) (end 208.364 120.523) (width 0.1524) (layer F.Cu) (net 3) (status 10))
 (segment (start 208.364 120.523) (end 206.713 122.174) (width 0.1524) (layer F.Cu) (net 3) (status 20))
 (segment (start 204.513 122.174) (end 201.991 122.174) (width 0.1524) (layer F.Cu) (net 19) (status 30))
 (segment (start 212.692 119.253) (end 207.094 119.253) (width 0.1524) (layer F.Cu) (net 2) (status 30))
 (segment (start 207.094 119.253) (end 206.713 119.634) (width 0.1524) (layer F.Cu) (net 2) (status 30))
 (segment (start 204.513 119.634) (end 201.864 119.634) (width 0.1524) (layer F.Cu) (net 20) (status 30))
 (segment (start 212.692 117.983) (end 207.475 117.983) (width 0.1524) (layer F.Cu) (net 1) (status 10))
 (segment (start 207.475 117.983) (end 206.713 117.221) (width 0.1524) (layer F.Cu) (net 1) (status 20))
 (segment (start 204.513 117.221) (end 201.864 117.221) (width 0.1524) (layer F.Cu) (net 21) (status 30))
 (segment (start 218.092 119.253) (end 220.345 119.253) (width 0.1524) (layer F.Cu) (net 14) (status 10))
 (segment (start 220.472 114.554) (end 206.713 114.554) (width 0.1524) (layer F.Cu) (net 14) (status 20))
 (segment (start 220.726 114.808) (end 220.472 114.554) (width 0.1524) (layer F.Cu) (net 14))
 (segment (start 220.726 118.872) (end 220.726 114.808) (width 0.1524) (layer F.Cu) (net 14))
 (segment (start 220.345 119.253) (end 220.726 118.872) (width 0.1524) (layer F.Cu) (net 14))
 (segment (start 204.513 114.554) (end 201.864 114.554) (width 0.1524) (layer F.Cu) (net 22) (status 30))
 (segment (start 231.775 117.541) (end 235.613 117.541) (width 0.1524) (layer F.Cu) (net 23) (status 30))
 (segment (start 235.613 117.541) (end 235.679 117.475) (width 0.1524) (layer F.Cu) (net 23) (status 30))
 (segment (start 228.092 113.538) (end 228.981 113.538) (width 0.1524) (layer F.Cu) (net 23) (status 10))
 (segment (start 231.775 116.332) (end 231.775 117.541) (width 0.1524) (layer F.Cu) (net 23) (status 20))
 (segment (start 228.981 113.538) (end 231.775 116.332) (width 0.1524) (layer F.Cu) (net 23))
 (segment (start 241.079 118.745) (end 242.763 118.745) (width 0.1524) (layer F.Cu) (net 24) (status 10))
 (segment (start 242.763 118.745) (end 244.287 120.269) (width 0.1524) (layer F.Cu) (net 24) (status 20))
 (segment (start 241.079 117.475) (end 244.033 117.475) (width 0.1524) (layer F.Cu) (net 25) (status 30))
 (segment (start 244.033 117.475) (end 244.287 117.729) (width 0.1524) (layer F.Cu) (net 25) (status 30))
 (segment (start 241.079 116.205) (end 243.144 116.205) (width 0.1524) (layer F.Cu) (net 26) (status 10))
 (segment (start 243.144 116.205) (end 244.287 115.062) (width 0.1524) (layer F.Cu) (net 26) (status 20))
 (segment (start 225.552 110.998) (end 225.552 110.744) (width 0.6096) (layer F.Cu) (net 27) (status 30))
 (segment (start 225.552 110.744) (end 225.933 110.363) (width 0.6096) (layer F.Cu) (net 27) (status 30))
 (segment (start 225.933 110.363) (end 246.507 110.363) (width 0.6096) (layer F.Cu) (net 27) (status 10))
 (segment (start 246.507 110.363) (end 248.158 112.014) (width 0.6096) (layer F.Cu) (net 27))
 (segment (start 248.158 112.014) (end 248.158 122.682) (width 0.6096) (layer F.Cu) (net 27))
 (segment (start 248.158 122.682) (end 245.425 125.415) (width 0.6096) (layer F.Cu) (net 27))
 (segment (start 245.425 125.415) (end 233.172 125.415) (width 0.6096) (layer F.Cu) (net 27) (status 20))
 (segment (start 233.172 127.315) (end 233.172 129.794) (width 0.1524) (layer F.Cu) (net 28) (status 30))
 (segment (start 233.172 129.794) (end 231.14 129.794) (width 0.1524) (layer F.Cu) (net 28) (status 10))
 (segment (start 226.822 130.048) (end 225.552 128.778) (width 0.1524) (layer F.Cu) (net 28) (status 20))
 (segment (start 230.886 130.048) (end 226.822 130.048) (width 0.1524) (layer F.Cu) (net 28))
 (segment (start 231.14 129.794) (end 230.886 130.048) (width 0.1524) (layer F.Cu) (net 28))
 (segment (start 236.662 133.985) (end 236.662 131.304) (width 0.1524) (layer F.Cu) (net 29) (status 10))
 (segment (start 236.662 131.304) (end 238.172 129.794) (width 0.1524) (layer F.Cu) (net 29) (status 20))
 (segment (start 238.172 129.794) (end 238.172 129.079) (width 0.1524) (layer B.Cu) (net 29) (status 30))
 (segment (start 238.172 129.079) (end 237.363 128.27) (width 0.1524) (layer B.Cu) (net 29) (status 10))
 (segment (start 237.363 128.27) (end 228.6 128.27) (width 0.1524) (layer B.Cu) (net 29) (status 20))
 (segment (start 228.6 128.27) (end 228.092 128.778) (width 0.1524) (layer B.Cu) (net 29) (status 30))
 (segment (start 218.092 124.333) (end 220.345 124.333) (width 0.1524) (layer F.Cu) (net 11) (status 10))
 (segment (start 226.822 117.348) (end 225.552 116.078) (width 0.1524) (layer F.Cu) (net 11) (status 20))
 (segment (start 226.822 121.92) (end 226.822 117.348) (width 0.1524) (layer F.Cu) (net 11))
 (segment (start 226.06 122.682) (end 226.822 121.92) (width 0.1524) (layer F.Cu) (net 11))
 (segment (start 221.996 122.682) (end 226.06 122.682) (width 0.1524) (layer F.Cu) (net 11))
 (segment (start 220.345 124.333) (end 221.996 122.682) (width 0.1524) (layer F.Cu) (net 11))
 (segment (start 218.092 120.523) (end 221.234 120.523) (width 0.1524) (layer F.Cu) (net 13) (status 10))
 (segment (start 225.552 120.523) (end 225.552 118.618) (width 0.1524) (layer B.Cu) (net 13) (status 20))
 (segment (start 221.234 120.523) (end 225.552 120.523) (width 0.1524) (layer B.Cu) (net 13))
 (via (at 221.234 120.523) (size 0.6858) (drill 0.3302) (layers F.Cu B.Cu) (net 13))
 (segment (start 225.552 126.238) (end 225.552 125.73) (width 0.1524) (layer F.Cu) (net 33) (status 30))
 (segment (start 225.552 125.73) (end 226.314 124.968) (width 0.1524) (layer F.Cu) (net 33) (status 10))
 (segment (start 226.314 124.968) (end 230.378 124.968) (width 0.1524) (layer F.Cu) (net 33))
 (segment (start 230.378 124.968) (end 232.283 123.063) (width 0.1524) (layer F.Cu) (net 33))
 (segment (start 232.283 123.063) (end 232.283 122.301) (width 0.1524) (layer F.Cu) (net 33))
 (segment (start 232.283 122.301) (end 233.299 121.285) (width 0.1524) (layer F.Cu) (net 33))
 (segment (start 233.299 121.285) (end 233.299 119.38) (width 0.1524) (layer F.Cu) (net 33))
 (via (at 233.299 119.38) (size 0.6858) (drill 0.3302) (layers F.Cu B.Cu) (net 33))
 (segment (start 233.299 119.38) (end 233.299 116.332) (width 0.1524) (layer B.Cu) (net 33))
 (via (at 233.299 116.332) (size 0.6858) (drill 0.3302) (layers F.Cu B.Cu) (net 33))
 (segment (start 233.299 116.332) (end 233.426 116.205) (width 0.1524) (layer F.Cu) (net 33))
 (segment (start 233.426 116.205) (end 235.679 116.205) (width 0.1524) (layer F.Cu) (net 33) (status 20))
 (segment (start 228.092 126.238) (end 231.013 126.238) (width 0.1524) (layer F.Cu) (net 34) (status 10))
 (segment (start 234.061 114.935) (end 235.679 114.935) (width 0.1524) (layer F.Cu) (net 34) (status 20))
 (via (at 234.061 114.935) (size 0.6858) (drill 0.3302) (layers F.Cu B.Cu) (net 34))
 (segment (start 234.061 118.364) (end 234.061 114.935) (width 0.1524) (layer B.Cu) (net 34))
 (via (at 234.061 118.364) (size 0.6858) (drill 0.3302) (layers F.Cu B.Cu) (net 34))
 (segment (start 234.061 121.92) (end 234.061 118.364) (width 0.1524) (layer F.Cu) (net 34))
 (segment (start 233.68 122.301) (end 234.061 121.92) (width 0.1524) (layer F.Cu) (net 34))
 (segment (start 233.68 122.682) (end 233.68 122.301) (width 0.1524) (layer F.Cu) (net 34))
 (segment (start 231.648 124.714) (end 233.68 122.682) (width 0.1524) (layer F.Cu) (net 34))
 (segment (start 231.648 125.603) (end 231.648 124.714) (width 0.1524) (layer F.Cu) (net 34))
 (segment (start 231.013 126.238) (end 231.648 125.603) (width 0.1524) (layer F.Cu) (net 34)))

